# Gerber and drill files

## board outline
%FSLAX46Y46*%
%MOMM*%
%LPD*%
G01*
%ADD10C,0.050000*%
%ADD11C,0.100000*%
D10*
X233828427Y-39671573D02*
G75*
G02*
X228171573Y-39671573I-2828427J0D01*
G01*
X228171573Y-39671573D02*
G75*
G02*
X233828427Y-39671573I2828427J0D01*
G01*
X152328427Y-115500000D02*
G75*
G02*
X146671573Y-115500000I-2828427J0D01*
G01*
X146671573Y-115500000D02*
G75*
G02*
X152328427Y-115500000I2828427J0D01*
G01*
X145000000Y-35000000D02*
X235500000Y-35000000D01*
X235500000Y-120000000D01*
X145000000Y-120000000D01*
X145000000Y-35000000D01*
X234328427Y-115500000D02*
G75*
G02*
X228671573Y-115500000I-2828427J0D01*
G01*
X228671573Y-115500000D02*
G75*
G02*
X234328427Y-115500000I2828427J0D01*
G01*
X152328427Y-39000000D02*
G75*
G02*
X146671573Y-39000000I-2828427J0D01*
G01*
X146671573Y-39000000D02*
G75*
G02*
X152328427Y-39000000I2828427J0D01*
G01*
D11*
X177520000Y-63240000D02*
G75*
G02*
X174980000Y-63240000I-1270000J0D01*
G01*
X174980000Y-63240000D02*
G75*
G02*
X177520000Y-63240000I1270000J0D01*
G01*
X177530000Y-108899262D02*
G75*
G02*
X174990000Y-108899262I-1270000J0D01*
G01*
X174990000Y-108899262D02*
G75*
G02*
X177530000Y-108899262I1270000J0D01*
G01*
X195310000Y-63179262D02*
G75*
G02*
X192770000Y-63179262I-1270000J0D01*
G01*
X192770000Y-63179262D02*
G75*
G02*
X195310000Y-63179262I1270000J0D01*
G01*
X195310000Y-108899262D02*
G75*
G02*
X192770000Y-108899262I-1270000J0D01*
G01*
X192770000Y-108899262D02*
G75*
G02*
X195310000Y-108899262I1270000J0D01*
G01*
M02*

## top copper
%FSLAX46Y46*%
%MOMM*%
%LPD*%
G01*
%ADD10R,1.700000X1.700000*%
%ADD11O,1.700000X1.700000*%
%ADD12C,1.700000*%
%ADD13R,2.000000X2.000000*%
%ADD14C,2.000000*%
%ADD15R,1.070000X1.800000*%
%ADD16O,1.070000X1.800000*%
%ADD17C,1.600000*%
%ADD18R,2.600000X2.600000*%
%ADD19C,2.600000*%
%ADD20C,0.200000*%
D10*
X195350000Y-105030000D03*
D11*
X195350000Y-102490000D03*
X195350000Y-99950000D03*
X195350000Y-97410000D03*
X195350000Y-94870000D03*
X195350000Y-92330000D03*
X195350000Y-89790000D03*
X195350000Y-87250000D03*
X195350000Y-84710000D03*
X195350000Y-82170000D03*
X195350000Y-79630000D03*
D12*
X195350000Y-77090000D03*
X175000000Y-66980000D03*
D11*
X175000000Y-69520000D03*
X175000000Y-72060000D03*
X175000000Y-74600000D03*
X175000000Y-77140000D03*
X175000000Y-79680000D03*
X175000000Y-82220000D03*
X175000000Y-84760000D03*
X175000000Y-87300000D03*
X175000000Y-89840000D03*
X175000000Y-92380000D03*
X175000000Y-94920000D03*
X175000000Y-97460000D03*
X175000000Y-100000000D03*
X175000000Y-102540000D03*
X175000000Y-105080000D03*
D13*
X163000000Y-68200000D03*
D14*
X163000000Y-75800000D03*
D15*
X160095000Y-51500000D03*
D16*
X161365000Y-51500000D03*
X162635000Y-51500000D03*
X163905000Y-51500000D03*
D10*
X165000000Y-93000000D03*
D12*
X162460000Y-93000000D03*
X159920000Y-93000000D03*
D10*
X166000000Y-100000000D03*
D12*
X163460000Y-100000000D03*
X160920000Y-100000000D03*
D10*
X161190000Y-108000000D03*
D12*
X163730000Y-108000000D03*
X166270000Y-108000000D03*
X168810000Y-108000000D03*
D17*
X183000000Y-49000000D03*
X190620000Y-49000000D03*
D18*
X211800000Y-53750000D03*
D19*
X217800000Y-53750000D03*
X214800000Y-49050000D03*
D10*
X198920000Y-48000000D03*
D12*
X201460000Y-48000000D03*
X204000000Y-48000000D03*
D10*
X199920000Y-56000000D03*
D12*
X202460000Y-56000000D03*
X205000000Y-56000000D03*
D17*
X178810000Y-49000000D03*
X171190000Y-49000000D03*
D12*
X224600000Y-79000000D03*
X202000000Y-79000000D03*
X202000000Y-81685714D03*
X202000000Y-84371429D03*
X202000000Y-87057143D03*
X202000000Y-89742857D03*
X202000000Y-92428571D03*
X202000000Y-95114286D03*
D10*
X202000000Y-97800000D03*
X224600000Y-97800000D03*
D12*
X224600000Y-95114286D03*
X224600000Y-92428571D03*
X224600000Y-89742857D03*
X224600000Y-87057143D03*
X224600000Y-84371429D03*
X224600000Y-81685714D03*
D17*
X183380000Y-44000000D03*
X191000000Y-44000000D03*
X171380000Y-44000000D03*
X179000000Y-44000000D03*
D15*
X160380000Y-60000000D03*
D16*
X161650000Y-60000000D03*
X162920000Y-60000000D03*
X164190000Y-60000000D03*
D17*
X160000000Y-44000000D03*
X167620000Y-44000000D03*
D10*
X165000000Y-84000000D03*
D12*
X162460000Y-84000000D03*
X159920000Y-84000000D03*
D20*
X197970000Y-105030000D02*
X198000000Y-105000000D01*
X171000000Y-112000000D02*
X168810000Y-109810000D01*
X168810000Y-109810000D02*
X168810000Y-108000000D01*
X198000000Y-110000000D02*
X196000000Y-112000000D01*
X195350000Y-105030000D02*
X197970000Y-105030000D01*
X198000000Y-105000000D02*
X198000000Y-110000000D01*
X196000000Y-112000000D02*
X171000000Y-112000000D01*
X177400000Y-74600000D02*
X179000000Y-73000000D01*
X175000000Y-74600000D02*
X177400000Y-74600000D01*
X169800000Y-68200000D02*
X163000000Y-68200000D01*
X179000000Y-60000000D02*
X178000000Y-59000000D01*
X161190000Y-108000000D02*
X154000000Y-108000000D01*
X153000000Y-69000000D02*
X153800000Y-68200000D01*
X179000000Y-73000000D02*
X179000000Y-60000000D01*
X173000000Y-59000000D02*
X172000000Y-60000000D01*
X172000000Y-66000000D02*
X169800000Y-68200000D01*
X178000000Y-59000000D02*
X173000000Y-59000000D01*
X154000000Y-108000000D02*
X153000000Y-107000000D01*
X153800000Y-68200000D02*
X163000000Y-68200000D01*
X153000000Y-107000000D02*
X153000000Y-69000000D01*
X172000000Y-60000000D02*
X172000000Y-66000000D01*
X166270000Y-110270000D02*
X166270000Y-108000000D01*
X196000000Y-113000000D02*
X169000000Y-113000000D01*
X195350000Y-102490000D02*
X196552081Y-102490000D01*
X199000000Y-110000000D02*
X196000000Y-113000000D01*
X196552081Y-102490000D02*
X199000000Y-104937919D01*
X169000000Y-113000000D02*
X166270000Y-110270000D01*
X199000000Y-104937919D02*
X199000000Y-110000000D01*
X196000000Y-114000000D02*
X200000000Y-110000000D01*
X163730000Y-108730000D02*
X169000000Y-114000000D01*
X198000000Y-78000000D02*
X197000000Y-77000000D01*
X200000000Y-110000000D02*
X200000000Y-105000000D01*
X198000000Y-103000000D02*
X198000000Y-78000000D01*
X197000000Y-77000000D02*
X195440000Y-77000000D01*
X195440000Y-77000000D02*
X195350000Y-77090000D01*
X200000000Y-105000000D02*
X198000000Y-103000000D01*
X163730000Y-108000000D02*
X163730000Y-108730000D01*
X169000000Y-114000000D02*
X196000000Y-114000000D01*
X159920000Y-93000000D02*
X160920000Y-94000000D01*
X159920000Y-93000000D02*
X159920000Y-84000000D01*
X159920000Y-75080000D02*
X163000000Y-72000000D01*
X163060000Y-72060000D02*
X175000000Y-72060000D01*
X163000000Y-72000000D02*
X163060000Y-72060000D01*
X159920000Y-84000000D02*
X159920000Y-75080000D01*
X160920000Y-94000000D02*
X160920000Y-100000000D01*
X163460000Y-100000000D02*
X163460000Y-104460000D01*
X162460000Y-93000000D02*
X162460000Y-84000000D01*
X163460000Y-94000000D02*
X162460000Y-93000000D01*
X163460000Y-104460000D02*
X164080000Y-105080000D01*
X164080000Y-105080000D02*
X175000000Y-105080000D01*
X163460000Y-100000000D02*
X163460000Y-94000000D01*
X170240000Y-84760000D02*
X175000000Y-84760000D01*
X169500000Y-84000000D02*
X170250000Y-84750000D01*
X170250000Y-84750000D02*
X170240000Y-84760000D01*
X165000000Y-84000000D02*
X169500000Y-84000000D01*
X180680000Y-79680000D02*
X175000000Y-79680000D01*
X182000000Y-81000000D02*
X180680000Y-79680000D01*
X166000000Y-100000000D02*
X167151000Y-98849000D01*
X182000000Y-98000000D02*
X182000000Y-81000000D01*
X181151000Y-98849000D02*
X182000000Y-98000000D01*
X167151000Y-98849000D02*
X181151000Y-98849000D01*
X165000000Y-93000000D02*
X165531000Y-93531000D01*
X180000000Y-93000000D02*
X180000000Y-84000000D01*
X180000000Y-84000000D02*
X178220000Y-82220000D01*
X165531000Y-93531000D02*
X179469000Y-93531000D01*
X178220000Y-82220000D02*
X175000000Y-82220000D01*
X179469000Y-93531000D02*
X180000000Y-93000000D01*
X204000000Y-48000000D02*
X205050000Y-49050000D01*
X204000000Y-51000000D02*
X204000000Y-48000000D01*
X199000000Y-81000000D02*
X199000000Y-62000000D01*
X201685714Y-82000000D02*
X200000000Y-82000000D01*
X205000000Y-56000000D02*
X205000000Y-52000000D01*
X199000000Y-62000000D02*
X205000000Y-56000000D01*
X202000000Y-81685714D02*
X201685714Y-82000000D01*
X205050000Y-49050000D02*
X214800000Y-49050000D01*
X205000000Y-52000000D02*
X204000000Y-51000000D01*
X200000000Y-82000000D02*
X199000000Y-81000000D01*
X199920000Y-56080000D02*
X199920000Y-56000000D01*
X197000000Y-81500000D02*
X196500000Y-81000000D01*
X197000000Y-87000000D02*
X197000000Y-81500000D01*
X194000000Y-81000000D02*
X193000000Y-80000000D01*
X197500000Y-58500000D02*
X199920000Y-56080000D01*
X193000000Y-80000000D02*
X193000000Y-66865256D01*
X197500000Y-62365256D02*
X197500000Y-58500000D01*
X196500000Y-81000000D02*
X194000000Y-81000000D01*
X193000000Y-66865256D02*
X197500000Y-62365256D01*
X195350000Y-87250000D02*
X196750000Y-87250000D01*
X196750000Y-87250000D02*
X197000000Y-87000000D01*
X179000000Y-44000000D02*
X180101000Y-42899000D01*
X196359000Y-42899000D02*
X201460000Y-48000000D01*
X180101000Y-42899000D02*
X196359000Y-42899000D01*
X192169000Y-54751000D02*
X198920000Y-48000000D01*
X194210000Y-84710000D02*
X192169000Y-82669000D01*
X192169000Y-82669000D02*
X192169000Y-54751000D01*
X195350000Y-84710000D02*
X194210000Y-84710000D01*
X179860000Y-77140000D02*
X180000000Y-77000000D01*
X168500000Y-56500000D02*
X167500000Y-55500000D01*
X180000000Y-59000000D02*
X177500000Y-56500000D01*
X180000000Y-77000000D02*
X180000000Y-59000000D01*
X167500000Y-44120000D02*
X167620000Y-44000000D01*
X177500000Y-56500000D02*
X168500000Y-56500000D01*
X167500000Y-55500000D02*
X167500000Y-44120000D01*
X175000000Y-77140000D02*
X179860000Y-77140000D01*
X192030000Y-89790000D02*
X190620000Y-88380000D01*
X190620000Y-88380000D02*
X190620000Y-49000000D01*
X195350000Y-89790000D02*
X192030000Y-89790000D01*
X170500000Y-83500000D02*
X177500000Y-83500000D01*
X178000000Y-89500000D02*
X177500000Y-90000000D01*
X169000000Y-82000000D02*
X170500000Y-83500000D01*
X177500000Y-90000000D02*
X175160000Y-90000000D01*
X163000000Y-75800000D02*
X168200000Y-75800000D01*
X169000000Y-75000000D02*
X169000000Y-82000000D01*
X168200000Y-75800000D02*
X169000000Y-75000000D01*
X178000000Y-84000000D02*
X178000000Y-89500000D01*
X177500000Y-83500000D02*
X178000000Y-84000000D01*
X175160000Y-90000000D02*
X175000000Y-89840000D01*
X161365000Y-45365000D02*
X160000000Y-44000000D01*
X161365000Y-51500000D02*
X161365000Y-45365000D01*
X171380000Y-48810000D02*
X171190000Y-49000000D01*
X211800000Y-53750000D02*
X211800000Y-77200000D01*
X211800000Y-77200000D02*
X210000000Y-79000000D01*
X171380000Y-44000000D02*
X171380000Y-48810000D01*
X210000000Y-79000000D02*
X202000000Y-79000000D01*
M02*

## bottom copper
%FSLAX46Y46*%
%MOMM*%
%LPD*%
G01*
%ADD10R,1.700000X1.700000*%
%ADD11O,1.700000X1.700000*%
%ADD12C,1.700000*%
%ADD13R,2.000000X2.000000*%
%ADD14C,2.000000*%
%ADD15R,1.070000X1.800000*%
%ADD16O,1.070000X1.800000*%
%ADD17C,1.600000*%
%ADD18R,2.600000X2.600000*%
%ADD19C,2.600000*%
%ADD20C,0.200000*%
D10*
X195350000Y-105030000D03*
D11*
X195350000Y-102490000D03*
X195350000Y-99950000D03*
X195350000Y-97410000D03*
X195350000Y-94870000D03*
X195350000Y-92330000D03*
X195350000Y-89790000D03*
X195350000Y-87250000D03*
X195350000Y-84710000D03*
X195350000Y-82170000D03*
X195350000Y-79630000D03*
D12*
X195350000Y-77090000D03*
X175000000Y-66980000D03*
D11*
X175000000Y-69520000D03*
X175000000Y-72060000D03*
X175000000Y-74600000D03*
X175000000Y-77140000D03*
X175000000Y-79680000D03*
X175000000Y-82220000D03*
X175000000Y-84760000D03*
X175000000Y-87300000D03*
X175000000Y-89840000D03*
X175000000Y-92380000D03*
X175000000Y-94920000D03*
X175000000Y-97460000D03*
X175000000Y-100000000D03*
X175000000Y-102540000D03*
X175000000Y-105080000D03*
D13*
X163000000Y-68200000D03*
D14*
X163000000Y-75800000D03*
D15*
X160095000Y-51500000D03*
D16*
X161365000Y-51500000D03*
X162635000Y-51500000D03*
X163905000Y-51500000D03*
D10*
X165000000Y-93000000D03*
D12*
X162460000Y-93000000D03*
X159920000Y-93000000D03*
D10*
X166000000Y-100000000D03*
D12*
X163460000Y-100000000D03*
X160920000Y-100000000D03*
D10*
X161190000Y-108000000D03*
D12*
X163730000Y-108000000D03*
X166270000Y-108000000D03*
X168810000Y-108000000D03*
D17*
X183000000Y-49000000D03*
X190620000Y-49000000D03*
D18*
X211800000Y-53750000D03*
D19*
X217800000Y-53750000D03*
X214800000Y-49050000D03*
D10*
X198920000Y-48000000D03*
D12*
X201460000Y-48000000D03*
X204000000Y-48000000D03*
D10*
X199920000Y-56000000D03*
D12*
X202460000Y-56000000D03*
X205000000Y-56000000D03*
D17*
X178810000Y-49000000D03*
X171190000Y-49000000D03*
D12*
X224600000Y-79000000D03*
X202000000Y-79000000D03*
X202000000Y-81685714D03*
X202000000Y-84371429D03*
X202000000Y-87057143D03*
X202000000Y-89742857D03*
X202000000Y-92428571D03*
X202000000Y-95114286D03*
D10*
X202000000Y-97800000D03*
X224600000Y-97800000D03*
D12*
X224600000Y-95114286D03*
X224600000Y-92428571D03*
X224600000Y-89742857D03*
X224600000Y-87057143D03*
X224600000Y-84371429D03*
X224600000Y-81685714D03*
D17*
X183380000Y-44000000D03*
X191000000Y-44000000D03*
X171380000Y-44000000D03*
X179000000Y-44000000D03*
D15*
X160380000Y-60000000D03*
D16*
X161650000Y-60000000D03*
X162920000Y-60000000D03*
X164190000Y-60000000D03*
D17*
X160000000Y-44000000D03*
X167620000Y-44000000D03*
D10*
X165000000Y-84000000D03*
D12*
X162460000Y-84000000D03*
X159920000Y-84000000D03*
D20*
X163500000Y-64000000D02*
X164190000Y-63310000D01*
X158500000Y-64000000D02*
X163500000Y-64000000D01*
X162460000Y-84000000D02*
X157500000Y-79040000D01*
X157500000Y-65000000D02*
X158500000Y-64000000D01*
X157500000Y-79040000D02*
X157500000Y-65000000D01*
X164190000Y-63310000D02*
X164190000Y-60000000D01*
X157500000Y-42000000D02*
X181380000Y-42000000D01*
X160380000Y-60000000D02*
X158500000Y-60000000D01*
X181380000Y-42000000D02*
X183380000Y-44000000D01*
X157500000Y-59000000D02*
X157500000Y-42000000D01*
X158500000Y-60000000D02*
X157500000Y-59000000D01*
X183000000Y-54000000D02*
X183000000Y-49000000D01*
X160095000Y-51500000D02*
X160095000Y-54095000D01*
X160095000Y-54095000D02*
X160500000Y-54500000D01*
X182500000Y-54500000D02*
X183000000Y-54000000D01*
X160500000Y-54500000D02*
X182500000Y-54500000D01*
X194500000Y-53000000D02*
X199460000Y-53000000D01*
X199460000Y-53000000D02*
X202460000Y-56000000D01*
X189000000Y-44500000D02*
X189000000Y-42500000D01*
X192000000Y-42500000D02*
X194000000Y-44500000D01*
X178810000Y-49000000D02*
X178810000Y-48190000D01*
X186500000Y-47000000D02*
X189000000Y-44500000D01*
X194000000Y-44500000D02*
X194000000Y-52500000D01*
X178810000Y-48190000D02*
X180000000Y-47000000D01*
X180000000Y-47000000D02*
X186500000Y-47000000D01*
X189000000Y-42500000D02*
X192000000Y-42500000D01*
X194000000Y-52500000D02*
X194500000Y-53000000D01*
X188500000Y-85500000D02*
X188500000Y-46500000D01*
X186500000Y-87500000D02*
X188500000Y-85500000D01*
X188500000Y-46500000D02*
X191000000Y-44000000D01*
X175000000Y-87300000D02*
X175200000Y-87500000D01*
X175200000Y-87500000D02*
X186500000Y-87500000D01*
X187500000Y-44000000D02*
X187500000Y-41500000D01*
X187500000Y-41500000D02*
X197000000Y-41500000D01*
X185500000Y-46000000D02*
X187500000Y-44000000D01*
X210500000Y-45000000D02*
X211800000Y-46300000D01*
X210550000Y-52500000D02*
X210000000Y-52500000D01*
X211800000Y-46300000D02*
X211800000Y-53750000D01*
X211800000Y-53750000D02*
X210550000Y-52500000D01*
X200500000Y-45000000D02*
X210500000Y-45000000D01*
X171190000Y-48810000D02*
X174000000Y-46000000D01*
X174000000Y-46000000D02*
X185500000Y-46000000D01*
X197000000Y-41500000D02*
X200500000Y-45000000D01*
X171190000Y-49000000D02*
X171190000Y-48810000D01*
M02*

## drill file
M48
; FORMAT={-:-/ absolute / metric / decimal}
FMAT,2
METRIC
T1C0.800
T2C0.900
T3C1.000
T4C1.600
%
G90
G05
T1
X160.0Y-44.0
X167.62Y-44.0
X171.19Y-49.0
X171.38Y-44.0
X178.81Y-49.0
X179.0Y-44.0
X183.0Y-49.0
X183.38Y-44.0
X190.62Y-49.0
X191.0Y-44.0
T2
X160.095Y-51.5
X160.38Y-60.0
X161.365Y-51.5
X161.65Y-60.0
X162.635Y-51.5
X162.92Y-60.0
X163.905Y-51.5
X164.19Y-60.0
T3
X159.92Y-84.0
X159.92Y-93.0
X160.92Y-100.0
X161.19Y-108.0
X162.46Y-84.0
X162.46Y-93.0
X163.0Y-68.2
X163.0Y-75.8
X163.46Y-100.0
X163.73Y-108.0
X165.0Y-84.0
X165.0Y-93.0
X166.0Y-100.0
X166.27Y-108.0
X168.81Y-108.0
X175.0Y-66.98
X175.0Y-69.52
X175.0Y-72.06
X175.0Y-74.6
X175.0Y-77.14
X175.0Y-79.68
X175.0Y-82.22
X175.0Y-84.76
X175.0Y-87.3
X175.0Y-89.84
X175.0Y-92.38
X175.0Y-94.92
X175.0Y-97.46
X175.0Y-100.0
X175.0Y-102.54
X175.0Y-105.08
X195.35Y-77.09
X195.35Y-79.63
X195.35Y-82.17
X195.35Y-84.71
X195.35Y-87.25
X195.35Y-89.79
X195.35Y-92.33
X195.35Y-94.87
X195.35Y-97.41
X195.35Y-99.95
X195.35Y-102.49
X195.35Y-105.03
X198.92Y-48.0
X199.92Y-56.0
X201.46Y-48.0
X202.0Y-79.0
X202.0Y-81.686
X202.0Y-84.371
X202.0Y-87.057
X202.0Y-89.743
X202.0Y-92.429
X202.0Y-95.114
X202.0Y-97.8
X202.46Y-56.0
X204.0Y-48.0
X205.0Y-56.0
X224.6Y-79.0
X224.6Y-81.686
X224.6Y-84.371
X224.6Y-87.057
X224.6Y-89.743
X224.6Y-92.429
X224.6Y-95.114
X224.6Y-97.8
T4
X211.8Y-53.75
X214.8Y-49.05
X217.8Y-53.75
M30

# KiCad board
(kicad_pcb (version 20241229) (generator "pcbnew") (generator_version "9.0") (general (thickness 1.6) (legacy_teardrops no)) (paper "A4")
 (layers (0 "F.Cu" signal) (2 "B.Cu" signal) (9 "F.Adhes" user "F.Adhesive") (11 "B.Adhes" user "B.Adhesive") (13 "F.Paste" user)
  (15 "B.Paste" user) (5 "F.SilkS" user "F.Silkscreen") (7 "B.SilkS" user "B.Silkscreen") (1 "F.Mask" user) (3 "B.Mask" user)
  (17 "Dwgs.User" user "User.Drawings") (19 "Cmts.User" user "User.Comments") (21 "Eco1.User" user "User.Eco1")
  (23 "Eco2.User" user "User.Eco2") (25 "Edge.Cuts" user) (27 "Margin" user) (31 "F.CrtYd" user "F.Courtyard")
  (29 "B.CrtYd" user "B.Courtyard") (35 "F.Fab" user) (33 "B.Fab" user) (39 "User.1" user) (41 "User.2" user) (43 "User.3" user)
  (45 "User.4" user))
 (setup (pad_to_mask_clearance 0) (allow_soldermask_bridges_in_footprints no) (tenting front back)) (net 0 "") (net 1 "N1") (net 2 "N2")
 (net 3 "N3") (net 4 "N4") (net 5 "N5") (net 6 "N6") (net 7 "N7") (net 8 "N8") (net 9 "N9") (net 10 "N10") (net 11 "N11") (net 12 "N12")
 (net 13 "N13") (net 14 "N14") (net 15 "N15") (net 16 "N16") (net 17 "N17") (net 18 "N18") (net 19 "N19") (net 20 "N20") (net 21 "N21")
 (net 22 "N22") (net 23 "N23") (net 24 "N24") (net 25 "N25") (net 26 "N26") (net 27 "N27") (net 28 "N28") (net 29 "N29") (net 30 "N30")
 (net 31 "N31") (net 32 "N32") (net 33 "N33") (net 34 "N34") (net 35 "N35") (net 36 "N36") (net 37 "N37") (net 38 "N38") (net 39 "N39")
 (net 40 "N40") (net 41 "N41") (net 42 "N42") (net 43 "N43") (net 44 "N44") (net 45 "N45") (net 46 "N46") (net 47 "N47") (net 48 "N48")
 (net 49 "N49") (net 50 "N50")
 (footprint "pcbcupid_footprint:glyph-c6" (layer "F.Cu") (at 185.168118 86.030247 -90)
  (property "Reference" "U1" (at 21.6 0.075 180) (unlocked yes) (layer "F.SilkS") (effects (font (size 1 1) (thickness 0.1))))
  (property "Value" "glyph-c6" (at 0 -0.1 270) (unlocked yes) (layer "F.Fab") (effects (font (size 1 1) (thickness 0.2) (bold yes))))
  (fp_circle (center -22.790247 8.918118) (end -21.520247 8.918118) (stroke (width 0.1) (type solid)) (fill no) (layer "Edge.Cuts"))
  (fp_circle (center 22.869015 8.908118) (end 24.139015 8.908118) (stroke (width 0.1) (type solid)) (fill no) (layer "Edge.Cuts"))
  (fp_circle (center -22.850985 -8.871882) (end -21.580985 -8.871882) (stroke (width 0.1) (type solid)) (fill no) (layer "Edge.Cuts"))
  (fp_circle (center 22.869015 -8.871882) (end 24.139015 -8.871882) (stroke (width 0.1) (type solid)) (fill no) (layer "Edge.Cuts"))
  (pad "1" thru_hole rect (at 18.999753 -10.181882 180) (size 1.7 1.7) (drill 1) (layers "*.Cu" "*.Mask") (remove_unused_layers no)
   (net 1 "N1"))
  (pad "2" thru_hole oval (at 16.459753 -10.181882 180) (size 1.7 1.7) (drill 1) (layers "*.Cu" "*.Mask") (remove_unused_layers no)
   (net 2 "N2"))
  (pad "3" thru_hole oval (at 13.919753 -10.181882 180) (size 1.7 1.7) (drill 1) (layers "*.Cu" "*.Mask") (remove_unused_layers no)
   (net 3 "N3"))
  (pad "4" thru_hole oval (at 11.379753 -10.181882 180) (size 1.7 1.7) (drill 1) (layers "*.Cu" "*.Mask") (remove_unused_layers no)
   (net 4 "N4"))
  (pad "5" thru_hole oval (at 8.839753 -10.181882 180) (size 1.7 1.7) (drill 1) (layers "*.Cu" "*.Mask") (remove_unused_layers no)
   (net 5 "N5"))
  (pad "6" thru_hole oval (at 6.299753 -10.181882 180) (size 1.7 1.7) (drill 1) (layers "*.Cu" "*.Mask") (remove_unused_layers no)
   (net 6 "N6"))
  (pad "7" thru_hole oval (at 3.759753 -10.181882 180) (size 1.7 1.7) (drill 1) (layers "*.Cu" "*.Mask") (remove_unused_layers no)
   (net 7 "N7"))
  (pad "8" thru_hole oval (at 1.219753 -10.181882 180) (size 1.7 1.7) (drill 1) (layers "*.Cu" "*.Mask") (remove_unused_layers no)
   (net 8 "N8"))
  (pad "9" thru_hole oval (at -1.320247 -10.181882 180) (size 1.7 1.7) (drill 1) (layers "*.Cu" "*.Mask") (remove_unused_layers no)
   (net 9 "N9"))
  (pad "10" thru_hole oval (at -3.860247 -10.181882 180) (size 1.7 1.7) (drill 1) (layers "*.Cu" "*.Mask") (remove_unused_layers no)
   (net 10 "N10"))
  (pad "11" thru_hole oval (at -6.400247 -10.181882 180) (size 1.7 1.7) (drill 1) (layers "*.Cu" "*.Mask") (remove_unused_layers no)
   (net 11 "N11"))
  (pad "12" thru_hole circle (at -8.940247 -10.181882 180) (size 1.7 1.7) (drill 1) (layers "*.Cu" "*.Mask") (remove_unused_layers no)
   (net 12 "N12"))
  (pad "13" thru_hole circle (at -19.050247 10.168118) (size 1.7 1.7) (drill 1) (layers "*.Cu" "*.Mask") (remove_unused_layers no)
   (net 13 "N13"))
  (pad "14" thru_hole oval (at -16.510247 10.168118) (size 1.7 1.7) (drill 1) (layers "*.Cu" "*.Mask") (remove_unused_layers no)
   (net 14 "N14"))
  (pad "15" thru_hole oval (at -13.970247 10.168118) (size 1.7 1.7) (drill 1) (layers "*.Cu" "*.Mask") (remove_unused_layers no)
   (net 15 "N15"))
  (pad "16" thru_hole oval (at -11.430247 10.168118) (size 1.7 1.7) (drill 1) (layers "*.Cu" "*.Mask") (remove_unused_layers no)
   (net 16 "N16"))
  (pad "17" thru_hole oval (at -8.890247 10.168118) (size 1.7 1.7) (drill 1) (layers "*.Cu" "*.Mask") (remove_unused_layers no)
   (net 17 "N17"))
  (pad "18" thru_hole oval (at -6.350247 10.168118) (size 1.7 1.7) (drill 1) (layers "*.Cu" "*.Mask") (remove_unused_layers no)
   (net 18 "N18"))
  (pad "19" thru_hole oval (at -3.810247 10.168118) (size 1.7 1.7) (drill 1) (layers "*.Cu" "*.Mask") (remove_unused_layers no)
   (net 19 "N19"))
  (pad "20" thru_hole oval (at -1.270247 10.168118) (size 1.7 1.7) (drill 1) (layers "*.Cu" "*.Mask") (remove_unused_layers no)
   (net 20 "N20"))
  (pad "21" thru_hole oval (at 1.269753 10.168118) (size 1.7 1.7) (drill 1) (layers "*.Cu" "*.Mask") (remove_unused_layers no)
   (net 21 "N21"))
  (pad "22" thru_hole oval (at 3.809753 10.168118) (size 1.7 1.7) (drill 1) (layers "*.Cu" "*.Mask") (remove_unused_layers no)
   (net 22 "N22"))
  (pad "23" thru_hole oval (at 6.349753 10.168118) (size 1.7 1.7) (drill 1) (layers "*.Cu" "*.Mask") (remove_unused_layers no)
   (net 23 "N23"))
  (pad "24" thru_hole oval (at 8.889753 10.168118) (size 1.7 1.7) (drill 1) (layers "*.Cu" "*.Mask") (remove_unused_layers no)
   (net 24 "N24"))
  (pad "25" thru_hole oval (at 11.429753 10.168118) (size 1.7 1.7) (drill 1) (layers "*.Cu" "*.Mask") (remove_unused_layers no)
   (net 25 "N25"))
  (pad "26" thru_hole oval (at 13.969753 10.168118) (size 1.7 1.7) (drill 1) (layers "*.Cu" "*.Mask") (remove_unused_layers no)
   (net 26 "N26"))
  (pad "27" thru_hole oval (at 16.509753 10.168118) (size 1.7 1.7) (drill 1) (layers "*.Cu" "*.Mask") (remove_unused_layers no)
   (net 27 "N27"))
  (pad "28" thru_hole oval (at 19.049753 10.168118) (size 1.7 1.7) (drill 1) (layers "*.Cu" "*.Mask") (remove_unused_layers no)
   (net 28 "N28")))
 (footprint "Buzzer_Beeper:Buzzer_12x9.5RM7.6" (layer "F.Cu") (at 163 68.2 -90)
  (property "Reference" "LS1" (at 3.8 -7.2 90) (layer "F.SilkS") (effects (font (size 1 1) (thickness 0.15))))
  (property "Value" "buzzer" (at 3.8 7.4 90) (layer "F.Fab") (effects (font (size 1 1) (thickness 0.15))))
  (pad "1" thru_hole rect (at 0 0 270) (size 2 2) (drill 1) (layers "*.Cu" "*.Mask") (remove_unused_layers no) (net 16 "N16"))
  (pad "2" thru_hole circle (at 7.6 0 270) (size 2 2) (drill 1) (layers "*.Cu" "*.Mask") (remove_unused_layers no) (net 22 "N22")))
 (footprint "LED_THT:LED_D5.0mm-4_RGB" (layer "F.Cu") (at 160.095 51.5)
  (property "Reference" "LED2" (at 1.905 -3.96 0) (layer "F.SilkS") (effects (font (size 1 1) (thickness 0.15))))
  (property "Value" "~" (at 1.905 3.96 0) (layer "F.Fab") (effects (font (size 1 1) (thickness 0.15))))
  (pad "1" thru_hole rect (at 0 0) (size 1.07 1.8) (drill 0.9) (layers "*.Cu" "*.Mask") (remove_unused_layers no) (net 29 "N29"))
  (pad "2" thru_hole oval (at 1.27 0) (size 1.07 1.8) (drill 0.9) (layers "*.Cu" "*.Mask") (remove_unused_layers no) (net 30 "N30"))
  (pad "3" thru_hole oval (at 2.54 0) (size 1.07 1.8) (drill 0.9) (layers "*.Cu" "*.Mask") (remove_unused_layers no))
  (pad "4" thru_hole oval (at 3.81 0) (size 1.07 1.8) (drill 0.9) (layers "*.Cu" "*.Mask") (remove_unused_layers no) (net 28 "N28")))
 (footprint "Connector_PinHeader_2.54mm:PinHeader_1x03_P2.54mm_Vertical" (layer "F.Cu") (at 165 93 -90)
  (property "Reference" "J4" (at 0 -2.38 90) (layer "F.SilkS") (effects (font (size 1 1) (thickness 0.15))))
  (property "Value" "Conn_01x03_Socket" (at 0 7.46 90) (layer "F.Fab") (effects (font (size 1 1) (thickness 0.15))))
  (pad "1" thru_hole rect (at 0 0 270) (size 1.7 1.7) (drill 1) (layers "*.Cu" "*.Mask") (remove_unused_layers no) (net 19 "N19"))
  (pad "2" thru_hole circle (at 0 2.54 270) (size 1.7 1.7) (drill 1) (layers "*.Cu" "*.Mask") (remove_unused_layers no) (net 28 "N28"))
  (pad "3" thru_hole circle (at 0 5.08 270) (size 1.7 1.7) (drill 1) (layers "*.Cu" "*.Mask") (remove_unused_layers no) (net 15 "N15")))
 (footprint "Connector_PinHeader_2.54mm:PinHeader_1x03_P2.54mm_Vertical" (layer "F.Cu") (at 166 100 -90)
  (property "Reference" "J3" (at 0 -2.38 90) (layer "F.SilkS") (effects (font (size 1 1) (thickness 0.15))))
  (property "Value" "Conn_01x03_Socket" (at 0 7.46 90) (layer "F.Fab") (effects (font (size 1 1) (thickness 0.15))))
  (pad "1" thru_hole rect (at 0 0 270) (size 1.7 1.7) (drill 1) (layers "*.Cu" "*.Mask") (remove_unused_layers no) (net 18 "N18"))
  (pad "2" thru_hole circle (at 0 2.54 270) (size 1.7 1.7) (drill 1) (layers "*.Cu" "*.Mask") (remove_unused_layers no) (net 28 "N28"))
  (pad "3" thru_hole circle (at 0 5.08 270) (size 1.7 1.7) (drill 1) (layers "*.Cu" "*.Mask") (remove_unused_layers no) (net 15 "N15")))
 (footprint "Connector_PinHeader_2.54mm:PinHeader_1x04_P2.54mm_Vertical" (layer "F.Cu") (at 161.19 108 90)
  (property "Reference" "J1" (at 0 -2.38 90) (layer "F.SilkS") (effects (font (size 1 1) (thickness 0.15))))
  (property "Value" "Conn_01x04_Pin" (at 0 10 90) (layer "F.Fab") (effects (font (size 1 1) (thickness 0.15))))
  (pad "1" thru_hole rect (at 0 0 90) (size 1.7 1.7) (drill 1) (layers "*.Cu" "*.Mask") (remove_unused_layers no) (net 16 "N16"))
  (pad "2" thru_hole circle (at 0 2.54 90) (size 1.7 1.7) (drill 1) (layers "*.Cu" "*.Mask") (remove_unused_layers no) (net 12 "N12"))
  (pad "3" thru_hole circle (at 0 5.08 90) (size 1.7 1.7) (drill 1) (layers "*.Cu" "*.Mask") (remove_unused_layers no) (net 2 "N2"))
  (pad "4" thru_hole circle (at 0 7.62 90) (size 1.7 1.7) (drill 1) (layers "*.Cu" "*.Mask") (remove_unused_layers no) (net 1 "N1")))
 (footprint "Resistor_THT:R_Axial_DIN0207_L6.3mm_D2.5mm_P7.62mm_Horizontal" (layer "F.Cu") (at 183 49)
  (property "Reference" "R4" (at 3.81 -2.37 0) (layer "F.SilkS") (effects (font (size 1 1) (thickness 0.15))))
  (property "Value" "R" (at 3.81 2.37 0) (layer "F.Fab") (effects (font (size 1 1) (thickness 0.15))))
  (pad "1" thru_hole circle (at 0 0) (size 1.6 1.6) (drill 0.8) (layers "*.Cu" "*.Mask") (remove_unused_layers no) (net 29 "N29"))
  (pad "2" thru_hole circle (at 7.62 0) (size 1.6 1.6) (drill 0.8) (layers "*.Cu" "*.Mask") (remove_unused_layers no) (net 7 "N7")))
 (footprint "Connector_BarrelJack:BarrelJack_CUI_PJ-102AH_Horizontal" (layer "F.Cu") (at 211.8 53.75 90)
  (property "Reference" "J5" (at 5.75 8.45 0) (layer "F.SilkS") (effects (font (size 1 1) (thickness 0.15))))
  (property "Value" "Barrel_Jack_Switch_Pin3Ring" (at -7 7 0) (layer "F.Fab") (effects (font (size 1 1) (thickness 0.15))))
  (pad "1" thru_hole rect (at 0 0 90) (size 2.6 2.6) (drill 1.6) (layers "*.Cu" "*.Mask") (remove_unused_layers no) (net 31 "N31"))
  (pad "2" thru_hole circle (at 0 6 90) (size 2.6 2.6) (drill 1.6) (layers "*.Cu" "*.Mask") (remove_unused_layers no) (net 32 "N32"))
  (pad "3" thru_hole circle (at 4.7 3 90) (size 2.6 2.6) (drill 1.6) (layers "*.Cu" "*.Mask") (remove_unused_layers no) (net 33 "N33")))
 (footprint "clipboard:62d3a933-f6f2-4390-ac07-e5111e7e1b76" (layer "F.Cu") (at 151 86)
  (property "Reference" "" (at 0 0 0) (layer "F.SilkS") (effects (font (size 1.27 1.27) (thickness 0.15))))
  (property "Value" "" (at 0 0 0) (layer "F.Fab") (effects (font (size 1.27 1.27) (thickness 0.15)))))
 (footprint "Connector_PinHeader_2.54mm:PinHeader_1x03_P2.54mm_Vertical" (layer "F.Cu") (at 198.92 48 90)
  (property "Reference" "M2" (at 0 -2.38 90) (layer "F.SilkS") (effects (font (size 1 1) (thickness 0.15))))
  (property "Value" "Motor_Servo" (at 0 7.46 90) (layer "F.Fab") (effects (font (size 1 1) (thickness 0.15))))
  (pad "1" thru_hole rect (at 0 0 90) (size 1.7 1.7) (drill 1) (layers "*.Cu" "*.Mask") (remove_unused_layers no) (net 9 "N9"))
  (pad "2" thru_hole circle (at 0 2.54 90) (size 1.7 1.7) (drill 1) (layers "*.Cu" "*.Mask") (remove_unused_layers no) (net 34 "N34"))
  (pad "3" thru_hole circle (at 0 5.08 90) (size 1.7 1.7) (drill 1) (layers "*.Cu" "*.Mask") (remove_unused_layers no) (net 33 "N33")))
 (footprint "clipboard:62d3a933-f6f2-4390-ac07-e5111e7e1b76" (layer "F.Cu") (at 148 89)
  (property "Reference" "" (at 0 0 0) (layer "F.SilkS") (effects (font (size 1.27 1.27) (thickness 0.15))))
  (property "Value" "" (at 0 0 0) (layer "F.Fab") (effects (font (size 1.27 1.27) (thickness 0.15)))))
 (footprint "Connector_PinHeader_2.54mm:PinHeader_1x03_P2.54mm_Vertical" (layer "F.Cu") (at 199.92 56 90)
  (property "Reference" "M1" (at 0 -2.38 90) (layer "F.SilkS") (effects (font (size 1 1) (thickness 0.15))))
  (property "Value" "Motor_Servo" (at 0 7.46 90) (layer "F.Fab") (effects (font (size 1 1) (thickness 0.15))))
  (pad "1" thru_hole rect (at 0 0 90) (size 1.7 1.7) (drill 1) (layers "*.Cu" "*.Mask") (remove_unused_layers no) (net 8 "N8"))
  (pad "2" thru_hole circle (at 0 2.54 90) (size 1.7 1.7) (drill 1) (layers "*.Cu" "*.Mask") (remove_unused_layers no) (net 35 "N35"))
  (pad "3" thru_hole circle (at 0 5.08 90) (size 1.7 1.7) (drill 1) (layers "*.Cu" "*.Mask") (remove_unused_layers no) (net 33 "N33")))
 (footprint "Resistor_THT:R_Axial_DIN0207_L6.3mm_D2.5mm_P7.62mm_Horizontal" (layer "F.Cu") (at 178.81 49 180)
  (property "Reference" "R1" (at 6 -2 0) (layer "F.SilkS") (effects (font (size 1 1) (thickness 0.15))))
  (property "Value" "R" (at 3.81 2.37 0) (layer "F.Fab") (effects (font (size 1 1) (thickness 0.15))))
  (pad "1" thru_hole circle (at 0 0 180) (size 1.6 1.6) (drill 0.8) (layers "*.Cu" "*.Mask") (remove_unused_layers no) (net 35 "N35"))
  (pad "2" thru_hole circle (at 7.62 0 180) (size 1.6 1.6) (drill 0.8) (layers "*.Cu" "*.Mask") (remove_unused_layers no) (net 31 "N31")))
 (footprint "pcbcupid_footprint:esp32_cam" (layer "F.Cu") (at 213 81.6)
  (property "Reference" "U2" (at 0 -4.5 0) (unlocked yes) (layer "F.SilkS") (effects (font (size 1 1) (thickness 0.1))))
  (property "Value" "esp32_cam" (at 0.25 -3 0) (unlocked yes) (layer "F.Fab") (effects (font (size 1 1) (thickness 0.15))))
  (pad "1" thru_hole circle (at 11.6 -2.6 180) (size 1.7 1.7) (drill 1) (layers "*.Cu" "*.Mask") (remove_unused_layers no) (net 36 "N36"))
  (pad "2" thru_hole circle (at -11 -2.6 180) (size 1.7 1.7) (drill 1) (layers "*.Cu" "*.Mask") (remove_unused_layers no) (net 31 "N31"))
  (pad "3" thru_hole circle (at -11 0.085714 180) (size 1.7 1.7) (drill 1) (layers "*.Cu" "*.Mask") (remove_unused_layers no) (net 33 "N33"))
  (pad "4" thru_hole circle (at -11 2.771429 180) (size 1.7 1.7) (drill 1) (layers "*.Cu" "*.Mask") (remove_unused_layers no) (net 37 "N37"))
  (pad "5" thru_hole circle (at -11 5.457143 180) (size 1.7 1.7) (drill 1) (layers "*.Cu" "*.Mask") (remove_unused_layers no) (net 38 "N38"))
  (pad "6" thru_hole circle (at -11 8.142857 180) (size 1.7 1.7) (drill 1) (layers "*.Cu" "*.Mask") (remove_unused_layers no) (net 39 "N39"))
  (pad "7" thru_hole circle (at -11 10.828571 180) (size 1.7 1.7) (drill 1) (layers "*.Cu" "*.Mask") (remove_unused_layers no)
   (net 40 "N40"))
  (pad "8" thru_hole circle (at -11 13.514286 180) (size 1.7 1.7) (drill 1) (layers "*.Cu" "*.Mask") (remove_unused_layers no)
   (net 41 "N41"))
  (pad "9" thru_hole rect (at -11 16.2 180) (size 1.7 1.7) (drill 1) (layers "*.Cu" "*.Mask") (remove_unused_layers no) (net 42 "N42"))
  (pad "10" thru_hole rect (at 11.6 16.2 180) (size 1.7 1.7) (drill 1) (layers "*.Cu" "*.Mask") (remove_unused_layers no) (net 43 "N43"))
  (pad "11" thru_hole circle (at 11.6 13.514286 180) (size 1.7 1.7) (drill 1) (layers "*.Cu" "*.Mask") (remove_unused_layers no)
   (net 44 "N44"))
  (pad "12" thru_hole circle (at 11.6 10.828571 180) (size 1.7 1.7) (drill 1) (layers "*.Cu" "*.Mask") (remove_unused_layers no)
   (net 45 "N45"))
  (pad "13" thru_hole circle (at 11.6 8.142857 180) (size 1.7 1.7) (drill 1) (layers "*.Cu" "*.Mask") (remove_unused_layers no)
   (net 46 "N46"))
  (pad "14" thru_hole circle (at 11.6 5.457143 180) (size 1.7 1.7) (drill 1) (layers "*.Cu" "*.Mask") (remove_unused_layers no))
  (pad "15" thru_hole circle (at 11.6 2.771429 180) (size 1.7 1.7) (drill 1) (layers "*.Cu" "*.Mask") (remove_unused_layers no))
  (pad "16" thru_hole circle (at 11.6 0.085714 180) (size 1.7 1.7) (drill 1) (layers "*.Cu" "*.Mask") (remove_unused_layers no)
   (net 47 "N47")))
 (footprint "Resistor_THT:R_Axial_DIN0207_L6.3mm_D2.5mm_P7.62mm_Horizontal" (layer "F.Cu") (at 183.38 44)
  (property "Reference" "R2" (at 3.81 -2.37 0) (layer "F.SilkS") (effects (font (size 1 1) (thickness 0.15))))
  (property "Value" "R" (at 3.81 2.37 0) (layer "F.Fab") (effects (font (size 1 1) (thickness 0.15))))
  (pad "1" thru_hole circle (at 0 0) (size 1.6 1.6) (drill 0.8) (layers "*.Cu" "*.Mask") (remove_unused_layers no) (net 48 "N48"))
  (pad "2" thru_hole circle (at 7.62 0) (size 1.6 1.6) (drill 0.8) (layers "*.Cu" "*.Mask") (remove_unused_layers no) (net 21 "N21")))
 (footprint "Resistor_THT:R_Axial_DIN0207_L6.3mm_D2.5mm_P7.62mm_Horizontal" (layer "F.Cu") (at 171.38 44)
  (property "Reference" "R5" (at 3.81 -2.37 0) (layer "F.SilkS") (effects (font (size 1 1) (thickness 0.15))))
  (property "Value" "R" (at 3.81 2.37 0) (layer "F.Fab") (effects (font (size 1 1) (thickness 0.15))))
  (pad "1" thru_hole circle (at 0 0) (size 1.6 1.6) (drill 0.8) (layers "*.Cu" "*.Mask") (remove_unused_layers no) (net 31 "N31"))
  (pad "2" thru_hole circle (at 7.62 0) (size 1.6 1.6) (drill 0.8) (layers "*.Cu" "*.Mask") (remove_unused_layers no) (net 34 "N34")))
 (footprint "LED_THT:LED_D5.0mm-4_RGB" (layer "F.Cu") (at 160.38 60)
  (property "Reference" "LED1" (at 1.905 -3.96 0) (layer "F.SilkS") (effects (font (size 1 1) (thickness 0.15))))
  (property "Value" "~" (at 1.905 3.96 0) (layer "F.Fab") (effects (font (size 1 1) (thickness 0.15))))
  (pad "1" thru_hole rect (at 0 0) (size 1.07 1.8) (drill 0.9) (layers "*.Cu" "*.Mask") (remove_unused_layers no) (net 48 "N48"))
  (pad "2" thru_hole oval (at 1.27 0) (size 1.07 1.8) (drill 0.9) (layers "*.Cu" "*.Mask") (remove_unused_layers no) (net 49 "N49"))
  (pad "3" thru_hole oval (at 2.54 0) (size 1.07 1.8) (drill 0.9) (layers "*.Cu" "*.Mask") (remove_unused_layers no) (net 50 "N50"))
  (pad "4" thru_hole oval (at 3.81 0) (size 1.07 1.8) (drill 0.9) (layers "*.Cu" "*.Mask") (remove_unused_layers no) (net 28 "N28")))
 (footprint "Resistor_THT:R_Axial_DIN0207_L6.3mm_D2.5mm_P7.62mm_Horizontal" (layer "F.Cu") (at 160 44)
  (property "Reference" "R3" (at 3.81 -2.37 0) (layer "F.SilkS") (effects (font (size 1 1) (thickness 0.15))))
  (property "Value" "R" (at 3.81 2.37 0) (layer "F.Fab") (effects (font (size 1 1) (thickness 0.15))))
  (pad "1" thru_hole circle (at 0 0) (size 1.6 1.6) (drill 0.8) (layers "*.Cu" "*.Mask") (remove_unused_layers no) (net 30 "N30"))
  (pad "2" thru_hole circle (at 7.62 0) (size 1.6 1.6) (drill 0.8) (layers "*.Cu" "*.Mask") (remove_unused_layers no) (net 17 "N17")))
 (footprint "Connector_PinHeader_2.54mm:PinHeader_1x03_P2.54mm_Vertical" (layer "F.Cu") (at 165 84 -90)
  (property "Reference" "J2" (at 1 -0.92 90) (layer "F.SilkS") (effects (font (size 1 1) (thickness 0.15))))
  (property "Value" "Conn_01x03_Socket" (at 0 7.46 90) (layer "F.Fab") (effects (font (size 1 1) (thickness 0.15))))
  (pad "1" thru_hole rect (at 0 0 270) (size 1.7 1.7) (drill 1) (layers "*.Cu" "*.Mask") (remove_unused_layers no) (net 20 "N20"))
  (pad "2" thru_hole circle (at 0 2.54 270) (size 1.7 1.7) (drill 1) (layers "*.Cu" "*.Mask") (remove_unused_layers no) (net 28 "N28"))
  (pad "3" thru_hole circle (at 0 5.08 270) (size 1.7 1.7) (drill 1) (layers "*.Cu" "*.Mask") (remove_unused_layers no) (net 15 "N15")))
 (gr_circle (center 231 39.671573) (end 229 41.671573) (stroke (width 0.05) (type default)) (fill no) (layer "Edge.Cuts"))
 (gr_circle (center 149.5 115.5) (end 147.5 117.5) (stroke (width 0.05) (type default)) (fill no) (layer "Edge.Cuts"))
 (gr_rect (start 145 35) (end 235.5 120) (stroke (width 0.05) (type default)) (fill no) (layer "Edge.Cuts"))
 (gr_circle (center 231.5 115.5) (end 229.5 117.5) (stroke (width 0.05) (type default)) (fill no) (layer "Edge.Cuts"))
 (gr_circle (center 149.5 39) (end 147.5 41) (stroke (width 0.05) (type default)) (fill no) (layer "Edge.Cuts"))
 (segment (start 197.97 105.03) (end 198 105) (width 0.2) (layer "F.Cu") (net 1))
 (segment (start 171 112) (end 168.81 109.81) (width 0.2) (layer "F.Cu") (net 1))
 (segment (start 168.81 109.81) (end 168.81 108) (width 0.2) (layer "F.Cu") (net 1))
 (segment (start 198 110) (end 196 112) (width 0.2) (layer "F.Cu") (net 1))
 (segment (start 195.35 105.03) (end 197.97 105.03) (width 0.2) (layer "F.Cu") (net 1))
 (segment (start 198 105) (end 198 110) (width 0.2) (layer "F.Cu") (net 1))
 (segment (start 196 112) (end 171 112) (width 0.2) (layer "F.Cu") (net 1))
 (segment (start 177.4 74.6) (end 179 73) (width 0.2) (layer "F.Cu") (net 16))
 (segment (start 175 74.6) (end 177.4 74.6) (width 0.2) (layer "F.Cu") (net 16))
 (segment (start 169.8 68.2) (end 163 68.2) (width 0.2) (layer "F.Cu") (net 16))
 (segment (start 179 60) (end 178 59) (width 0.2) (layer "F.Cu") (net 16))
 (segment (start 161.19 108) (end 154 108) (width 0.2) (layer "F.Cu") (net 16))
 (segment (start 153 69) (end 153.8 68.2) (width 0.2) (layer "F.Cu") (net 16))
 (segment (start 179 73) (end 179 60) (width 0.2) (layer "F.Cu") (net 16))
 (segment (start 173 59) (end 172 60) (width 0.2) (layer "F.Cu") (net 16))
 (segment (start 172 66) (end 169.8 68.2) (width 0.2) (layer "F.Cu") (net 16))
 (segment (start 178 59) (end 173 59) (width 0.2) (layer "F.Cu") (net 16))
 (segment (start 154 108) (end 153 107) (width 0.2) (layer "F.Cu") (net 16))
 (segment (start 153.8 68.2) (end 163 68.2) (width 0.2) (layer "F.Cu") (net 16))
 (segment (start 153 107) (end 153 69) (width 0.2) (layer "F.Cu") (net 16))
 (segment (start 172 60) (end 172 66) (width 0.2) (layer "F.Cu") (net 16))
 (segment (start 166.27 110.27) (end 166.27 108) (width 0.2) (layer "F.Cu") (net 2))
 (segment (start 196 113) (end 169 113) (width 0.2) (layer "F.Cu") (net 2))
 (segment (start 195.35 102.49) (end 196.552081 102.49) (width 0.2) (layer "F.Cu") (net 2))
 (segment (start 199 110) (end 196 113) (width 0.2) (layer "F.Cu") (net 2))
 (segment (start 196.552081 102.49) (end 199 104.937919) (width 0.2) (layer "F.Cu") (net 2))
 (segment (start 169 113) (end 166.27 110.27) (width 0.2) (layer "F.Cu") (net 2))
 (segment (start 199 104.937919) (end 199 110) (width 0.2) (layer "F.Cu") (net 2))
 (segment (start 196 114) (end 200 110) (width 0.2) (layer "F.Cu") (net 12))
 (segment (start 163.73 108.73) (end 169 114) (width 0.2) (layer "F.Cu") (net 12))
 (segment (start 198 78) (end 197 77) (width 0.2) (layer "F.Cu") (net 12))
 (segment (start 200 110) (end 200 105) (width 0.2) (layer "F.Cu") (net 12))
 (segment (start 198 103) (end 198 78) (width 0.2) (layer "F.Cu") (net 12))
 (segment (start 197 77) (end 195.44 77) (width 0.2) (layer "F.Cu") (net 12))
 (segment (start 195.44 77) (end 195.35 77.09) (width 0.2) (layer "F.Cu") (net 12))
 (segment (start 200 105) (end 198 103) (width 0.2) (layer "F.Cu") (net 12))
 (segment (start 163.73 108) (end 163.73 108.73) (width 0.2) (layer "F.Cu") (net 12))
 (segment (start 169 114) (end 196 114) (width 0.2) (layer "F.Cu") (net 12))
 (segment (start 159.92 93) (end 160.92 94) (width 0.2) (layer "F.Cu") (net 15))
 (segment (start 159.92 93) (end 159.92 84) (width 0.2) (layer "F.Cu") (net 15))
 (segment (start 159.92 75.08) (end 163 72) (width 0.2) (layer "F.Cu") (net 15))
 (segment (start 163.06 72.06) (end 175 72.06) (width 0.2) (layer "F.Cu") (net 15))
 (segment (start 163 72) (end 163.06 72.06) (width 0.2) (layer "F.Cu") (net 15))
 (segment (start 159.92 84) (end 159.92 75.08) (width 0.2) (layer "F.Cu") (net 15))
 (segment (start 160.92 94) (end 160.92 100) (width 0.2) (layer "F.Cu") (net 15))
 (segment (start 163.46 100) (end 163.46 104.46) (width 0.2) (layer "F.Cu") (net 28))
 (segment (start 162.46 93) (end 162.46 84) (width 0.2) (layer "F.Cu") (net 28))
 (segment (start 163.46 94) (end 162.46 93) (width 0.2) (layer "F.Cu") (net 28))
 (segment (start 163.46 104.46) (end 164.08 105.08) (width 0.2) (layer "F.Cu") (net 28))
 (segment (start 164.08 105.08) (end 175 105.08) (width 0.2) (layer "F.Cu") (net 28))
 (segment (start 163.46 100) (end 163.46 94) (width 0.2) (layer "F.Cu") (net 28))
 (segment (start 163.5 64) (end 164.19 63.31) (width 0.2) (layer "B.Cu") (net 28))
 (segment (start 158.5 64) (end 163.5 64) (width 0.2) (layer "B.Cu") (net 28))
 (segment (start 162.46 84) (end 157.5 79.04) (width 0.2) (layer "B.Cu") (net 28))
 (segment (start 157.5 65) (end 158.5 64) (width 0.2) (layer "B.Cu") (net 28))
 (segment (start 157.5 79.04) (end 157.5 65) (width 0.2) (layer "B.Cu") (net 28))
 (segment (start 164.19 63.31) (end 164.19 60) (width 0.2) (layer "B.Cu") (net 28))
 (segment (start 170.24 84.76) (end 175 84.76) (width 0.2) (layer "F.Cu") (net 20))
 (segment (start 169.5 84) (end 170.25 84.75) (width 0.2) (layer "F.Cu") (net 20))
 (segment (start 170.25 84.75) (end 170.24 84.76) (width 0.2) (layer "F.Cu") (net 20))
 (segment (start 165 84) (end 169.5 84) (width 0.2) (layer "F.Cu") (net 20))
 (segment (start 180.68 79.68) (end 175 79.68) (width 0.2) (layer "F.Cu") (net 18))
 (segment (start 182 81) (end 180.68 79.68) (width 0.2) (layer "F.Cu") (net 18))
 (segment (start 166 100) (end 167.151 98.849) (width 0.2) (layer "F.Cu") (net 18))
 (segment (start 182 98) (end 182 81) (width 0.2) (layer "F.Cu") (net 18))
 (segment (start 181.151 98.849) (end 182 98) (width 0.2) (layer "F.Cu") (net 18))
 (segment (start 167.151 98.849) (end 181.151 98.849) (width 0.2) (layer "F.Cu") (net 18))
 (segment (start 165 93) (end 165.531 93.531) (width 0.2) (layer "F.Cu") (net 19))
 (segment (start 180 93) (end 180 84) (width 0.2) (layer "F.Cu") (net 19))
 (segment (start 180 84) (end 178.22 82.22) (width 0.2) (layer "F.Cu") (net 19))
 (segment (start 165.531 93.531) (end 179.469 93.531) (width 0.2) (layer "F.Cu") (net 19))
 (segment (start 178.22 82.22) (end 175 82.22) (width 0.2) (layer "F.Cu") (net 19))
 (segment (start 179.469 93.531) (end 180 93) (width 0.2) (layer "F.Cu") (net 19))
 (segment (start 204 48) (end 205.05 49.05) (width 0.2) (layer "F.Cu") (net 33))
 (segment (start 204 51) (end 204 48) (width 0.2) (layer "F.Cu") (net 33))
 (segment (start 199 81) (end 199 62) (width 0.2) (layer "F.Cu") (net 33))
 (segment (start 201.685714 82) (end 200 82) (width 0.2) (layer "F.Cu") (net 33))
 (segment (start 205 56) (end 205 52) (width 0.2) (layer "F.Cu") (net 33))
 (segment (start 199 62) (end 205 56) (width 0.2) (layer "F.Cu") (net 33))
 (segment (start 202 81.685714) (end 201.685714 82) (width 0.2) (layer "F.Cu") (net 33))
 (segment (start 205.05 49.05) (end 214.8 49.05) (width 0.2) (layer "F.Cu") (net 33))
 (segment (start 205 52) (end 204 51) (width 0.2) (layer "F.Cu") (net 33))
 (segment (start 200 82) (end 199 81) (width 0.2) (layer "F.Cu") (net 33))
 (segment (start 157.5 42) (end 181.38 42) (width 0.2) (layer "B.Cu") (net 48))
 (segment (start 160.38 60) (end 158.5 60) (width 0.2) (layer "B.Cu") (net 48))
 (segment (start 181.38 42) (end 183.38 44) (width 0.2) (layer "B.Cu") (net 48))
 (segment (start 157.5 59) (end 157.5 42) (width 0.2) (layer "B.Cu") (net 48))
 (segment (start 158.5 60) (end 157.5 59) (width 0.2) (layer "B.Cu") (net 48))
 (segment (start 183 54) (end 183 49) (width 0.2) (layer "B.Cu") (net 29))
 (segment (start 160.095 51.5) (end 160.095 54.095) (width 0.2) (layer "B.Cu") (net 29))
 (segment (start 160.095 54.095) (end 160.5 54.5) (width 0.2) (layer "B.Cu") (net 29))
 (segment (start 182.5 54.5) (end 183 54) (width 0.2) (layer "B.Cu") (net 29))
 (segment (start 160.5 54.5) (end 182.5 54.5) (width 0.2) (layer "B.Cu") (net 29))
 (segment (start 194.5 53) (end 199.46 53) (width 0.2) (layer "B.Cu") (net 35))
 (segment (start 199.46 53) (end 202.46 56) (width 0.2) (layer "B.Cu") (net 35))
 (segment (start 189 44.5) (end 189 42.5) (width 0.2) (layer "B.Cu") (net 35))
 (segment (start 192 42.5) (end 194 44.5) (width 0.2) (layer "B.Cu") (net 35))
 (segment (start 178.81 49) (end 178.81 48.19) (width 0.2) (layer "B.Cu") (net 35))
 (segment (start 186.5 47) (end 189 44.5) (width 0.2) (layer "B.Cu") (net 35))
 (segment (start 194 44.5) (end 194 52.5) (width 0.2) (layer "B.Cu") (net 35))
 (segment (start 178.81 48.19) (end 180 47) (width 0.2) (layer "B.Cu") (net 35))
 (segment (start 180 47) (end 186.5 47) (width 0.2) (layer "B.Cu") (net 35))
 (segment (start 189 42.5) (end 192 42.5) (width 0.2) (layer "B.Cu") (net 35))
 (segment (start 194 52.5) (end 194.5 53) (width 0.2) (layer "B.Cu") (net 35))
 (segment (start 199.92 56.08) (end 199.92 56) (width 0.2) (layer "F.Cu") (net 8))
 (segment (start 197 81.5) (end 196.5 81) (width 0.2) (layer "F.Cu") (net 8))
 (segment (start 197 87) (end 197 81.5) (width 0.2) (layer "F.Cu") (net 8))
 (segment (start 194 81) (end 193 80) (width 0.2) (layer "F.Cu") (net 8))
 (segment (start 197.5 58.5) (end 199.92 56.08) (width 0.2) (layer "F.Cu") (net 8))
 (segment (start 193 80) (end 193 66.865256) (width 0.2) (layer "F.Cu") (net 8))
 (segment (start 197.5 62.365256) (end 197.5 58.5) (width 0.2) (layer "F.Cu") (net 8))
 (segment (start 196.5 81) (end 194 81) (width 0.2) (layer "F.Cu") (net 8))
 (segment (start 193 66.865256) (end 197.5 62.365256) (width 0.2) (layer "F.Cu") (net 8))
 (segment (start 195.35 87.25) (end 196.75 87.25) (width 0.2) (layer "F.Cu") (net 8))
 (segment (start 196.75 87.25) (end 197 87) (width 0.2) (layer "F.Cu") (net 8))
 (segment (start 179 44) (end 180.101 42.899) (width 0.2) (layer "F.Cu") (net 34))
 (segment (start 196.359 42.899) (end 201.46 48) (width 0.2) (layer "F.Cu") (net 34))
 (segment (start 180.101 42.899) (end 196.359 42.899) (width 0.2) (layer "F.Cu") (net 34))
 (segment (start 192.169 54.751) (end 198.92 48) (width 0.2) (layer "F.Cu") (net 9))
 (segment (start 194.21 84.71) (end 192.169 82.669) (width 0.2) (layer "F.Cu") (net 9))
 (segment (start 192.169 82.669) (end 192.169 54.751) (width 0.2) (layer "F.Cu") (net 9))
 (segment (start 195.35 84.71) (end 194.21 84.71) (width 0.2) (layer "F.Cu") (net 9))
 (segment (start 188.5 85.5) (end 188.5 46.5) (width 0.2) (layer "B.Cu") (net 21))
 (segment (start 186.5 87.5) (end 188.5 85.5) (width 0.2) (layer "B.Cu") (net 21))
 (segment (start 188.5 46.5) (end 191 44) (width 0.2) (layer "B.Cu") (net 21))
 (segment (start 175 87.3) (end 175.2 87.5) (width 0.2) (layer "B.Cu") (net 21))
 (segment (start 175.2 87.5) (end 186.5 87.5) (width 0.2) (layer "B.Cu") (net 21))
 (segment (start 179.86 77.14) (end 180 77) (width 0.2) (layer "F.Cu") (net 17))
 (segment (start 168.5 56.5) (end 167.5 55.5) (width 0.2) (layer "F.Cu") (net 17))
 (segment (start 180 59) (end 177.5 56.5) (width 0.2) (layer "F.Cu") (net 17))
 (segment (start 180 77) (end 180 59) (width 0.2) (layer "F.Cu") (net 17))
 (segment (start 167.5 44.12) (end 167.62 44) (width 0.2) (layer "F.Cu") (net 17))
 (segment (start 177.5 56.5) (end 168.5 56.5) (width 0.2) (layer "F.Cu") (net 17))
 (segment (start 167.5 55.5) (end 167.5 44.12) (width 0.2) (layer "F.Cu") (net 17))
 (segment (start 175 77.14) (end 179.86 77.14) (width 0.2) (layer "F.Cu") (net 17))
 (segment (start 192.03 89.79) (end 190.62 88.38) (width 0.2) (layer "F.Cu") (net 7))
 (segment (start 190.62 88.38) (end 190.62 49) (width 0.2) (layer "F.Cu") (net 7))
 (segment (start 195.35 89.79) (end 192.03 89.79) (width 0.2) (layer "F.Cu") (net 7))
 (segment (start 170.5 83.5) (end 177.5 83.5) (width 0.2) (layer "F.Cu") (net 22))
 (segment (start 178 89.5) (end 177.5 90) (width 0.2) (layer "F.Cu") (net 22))
 (segment (start 169 82) (end 170.5 83.5) (width 0.2) (layer "F.Cu") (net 22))
 (segment (start 177.5 90) (end 175.16 90) (width 0.2) (layer "F.Cu") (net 22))
 (segment (start 163 75.8) (end 168.2 75.8) (width 0.2) (layer "F.Cu") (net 22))
 (segment (start 169 75) (end 169 82) (width 0.2) (layer "F.Cu") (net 22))
 (segment (start 168.2 75.8) (end 169 75) (width 0.2) (layer "F.Cu") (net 22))
 (segment (start 178 84) (end 178 89.5) (width 0.2) (layer "F.Cu") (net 22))
 (segment (start 177.5 83.5) (end 178 84) (width 0.2) (layer "F.Cu") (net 22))
 (segment (start 175.16 90) (end 175 89.84) (width 0.2) (layer "F.Cu") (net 22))
 (segment (start 161.365 45.365) (end 160 44) (width 0.2) (layer "F.Cu") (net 30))
 (segment (start 161.365 51.5) (end 161.365 45.365) (width 0.2) (layer "F.Cu") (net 30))
 (segment (start 171.38 48.81) (end 171.19 49) (width 0.2) (layer "F.Cu") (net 31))
 (segment (start 211.8 53.75) (end 211.8 77.2) (width 0.2) (layer "F.Cu") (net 31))
 (segment (start 211.8 77.2) (end 210 79) (width 0.2) (layer "F.Cu") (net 31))
 (segment (start 171.38 44) (end 171.38 48.81) (width 0.2) (layer "F.Cu") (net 31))
 (segment (start 210 79) (end 202 79) (width 0.2) (layer "F.Cu") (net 31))
 (segment (start 187.5 44) (end 187.5 41.5) (width 0.2) (layer "B.Cu") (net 31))
 (segment (start 187.5 41.5) (end 197 41.5) (width 0.2) (layer "B.Cu") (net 31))
 (segment (start 185.5 46) (end 187.5 44) (width 0.2) (layer "B.Cu") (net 31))
 (segment (start 210.5 45) (end 211.8 46.3) (width 0.2) (layer "B.Cu") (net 31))
 (segment (start 210.55 52.5) (end 210 52.5) (width 0.2) (layer "B.Cu") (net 31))
 (segment (start 211.8 46.3) (end 211.8 53.75) (width 0.2) (layer "B.Cu") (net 31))
 (segment (start 211.8 53.75) (end 210.55 52.5) (width 0.2) (layer "B.Cu") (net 31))
 (segment (start 200.5 45) (end 210.5 45) (width 0.2) (layer "B.Cu") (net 31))
 (segment (start 171.19 48.81) (end 174 46) (width 0.2) (layer "B.Cu") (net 31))
 (segment (start 174 46) (end 185.5 46) (width 0.2) (layer "B.Cu") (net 31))
 (segment (start 197 41.5) (end 200.5 45) (width 0.2) (layer "B.Cu") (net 31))
 (segment (start 171.19 49) (end 171.19 48.81) (width 0.2) (layer "B.Cu") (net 31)))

